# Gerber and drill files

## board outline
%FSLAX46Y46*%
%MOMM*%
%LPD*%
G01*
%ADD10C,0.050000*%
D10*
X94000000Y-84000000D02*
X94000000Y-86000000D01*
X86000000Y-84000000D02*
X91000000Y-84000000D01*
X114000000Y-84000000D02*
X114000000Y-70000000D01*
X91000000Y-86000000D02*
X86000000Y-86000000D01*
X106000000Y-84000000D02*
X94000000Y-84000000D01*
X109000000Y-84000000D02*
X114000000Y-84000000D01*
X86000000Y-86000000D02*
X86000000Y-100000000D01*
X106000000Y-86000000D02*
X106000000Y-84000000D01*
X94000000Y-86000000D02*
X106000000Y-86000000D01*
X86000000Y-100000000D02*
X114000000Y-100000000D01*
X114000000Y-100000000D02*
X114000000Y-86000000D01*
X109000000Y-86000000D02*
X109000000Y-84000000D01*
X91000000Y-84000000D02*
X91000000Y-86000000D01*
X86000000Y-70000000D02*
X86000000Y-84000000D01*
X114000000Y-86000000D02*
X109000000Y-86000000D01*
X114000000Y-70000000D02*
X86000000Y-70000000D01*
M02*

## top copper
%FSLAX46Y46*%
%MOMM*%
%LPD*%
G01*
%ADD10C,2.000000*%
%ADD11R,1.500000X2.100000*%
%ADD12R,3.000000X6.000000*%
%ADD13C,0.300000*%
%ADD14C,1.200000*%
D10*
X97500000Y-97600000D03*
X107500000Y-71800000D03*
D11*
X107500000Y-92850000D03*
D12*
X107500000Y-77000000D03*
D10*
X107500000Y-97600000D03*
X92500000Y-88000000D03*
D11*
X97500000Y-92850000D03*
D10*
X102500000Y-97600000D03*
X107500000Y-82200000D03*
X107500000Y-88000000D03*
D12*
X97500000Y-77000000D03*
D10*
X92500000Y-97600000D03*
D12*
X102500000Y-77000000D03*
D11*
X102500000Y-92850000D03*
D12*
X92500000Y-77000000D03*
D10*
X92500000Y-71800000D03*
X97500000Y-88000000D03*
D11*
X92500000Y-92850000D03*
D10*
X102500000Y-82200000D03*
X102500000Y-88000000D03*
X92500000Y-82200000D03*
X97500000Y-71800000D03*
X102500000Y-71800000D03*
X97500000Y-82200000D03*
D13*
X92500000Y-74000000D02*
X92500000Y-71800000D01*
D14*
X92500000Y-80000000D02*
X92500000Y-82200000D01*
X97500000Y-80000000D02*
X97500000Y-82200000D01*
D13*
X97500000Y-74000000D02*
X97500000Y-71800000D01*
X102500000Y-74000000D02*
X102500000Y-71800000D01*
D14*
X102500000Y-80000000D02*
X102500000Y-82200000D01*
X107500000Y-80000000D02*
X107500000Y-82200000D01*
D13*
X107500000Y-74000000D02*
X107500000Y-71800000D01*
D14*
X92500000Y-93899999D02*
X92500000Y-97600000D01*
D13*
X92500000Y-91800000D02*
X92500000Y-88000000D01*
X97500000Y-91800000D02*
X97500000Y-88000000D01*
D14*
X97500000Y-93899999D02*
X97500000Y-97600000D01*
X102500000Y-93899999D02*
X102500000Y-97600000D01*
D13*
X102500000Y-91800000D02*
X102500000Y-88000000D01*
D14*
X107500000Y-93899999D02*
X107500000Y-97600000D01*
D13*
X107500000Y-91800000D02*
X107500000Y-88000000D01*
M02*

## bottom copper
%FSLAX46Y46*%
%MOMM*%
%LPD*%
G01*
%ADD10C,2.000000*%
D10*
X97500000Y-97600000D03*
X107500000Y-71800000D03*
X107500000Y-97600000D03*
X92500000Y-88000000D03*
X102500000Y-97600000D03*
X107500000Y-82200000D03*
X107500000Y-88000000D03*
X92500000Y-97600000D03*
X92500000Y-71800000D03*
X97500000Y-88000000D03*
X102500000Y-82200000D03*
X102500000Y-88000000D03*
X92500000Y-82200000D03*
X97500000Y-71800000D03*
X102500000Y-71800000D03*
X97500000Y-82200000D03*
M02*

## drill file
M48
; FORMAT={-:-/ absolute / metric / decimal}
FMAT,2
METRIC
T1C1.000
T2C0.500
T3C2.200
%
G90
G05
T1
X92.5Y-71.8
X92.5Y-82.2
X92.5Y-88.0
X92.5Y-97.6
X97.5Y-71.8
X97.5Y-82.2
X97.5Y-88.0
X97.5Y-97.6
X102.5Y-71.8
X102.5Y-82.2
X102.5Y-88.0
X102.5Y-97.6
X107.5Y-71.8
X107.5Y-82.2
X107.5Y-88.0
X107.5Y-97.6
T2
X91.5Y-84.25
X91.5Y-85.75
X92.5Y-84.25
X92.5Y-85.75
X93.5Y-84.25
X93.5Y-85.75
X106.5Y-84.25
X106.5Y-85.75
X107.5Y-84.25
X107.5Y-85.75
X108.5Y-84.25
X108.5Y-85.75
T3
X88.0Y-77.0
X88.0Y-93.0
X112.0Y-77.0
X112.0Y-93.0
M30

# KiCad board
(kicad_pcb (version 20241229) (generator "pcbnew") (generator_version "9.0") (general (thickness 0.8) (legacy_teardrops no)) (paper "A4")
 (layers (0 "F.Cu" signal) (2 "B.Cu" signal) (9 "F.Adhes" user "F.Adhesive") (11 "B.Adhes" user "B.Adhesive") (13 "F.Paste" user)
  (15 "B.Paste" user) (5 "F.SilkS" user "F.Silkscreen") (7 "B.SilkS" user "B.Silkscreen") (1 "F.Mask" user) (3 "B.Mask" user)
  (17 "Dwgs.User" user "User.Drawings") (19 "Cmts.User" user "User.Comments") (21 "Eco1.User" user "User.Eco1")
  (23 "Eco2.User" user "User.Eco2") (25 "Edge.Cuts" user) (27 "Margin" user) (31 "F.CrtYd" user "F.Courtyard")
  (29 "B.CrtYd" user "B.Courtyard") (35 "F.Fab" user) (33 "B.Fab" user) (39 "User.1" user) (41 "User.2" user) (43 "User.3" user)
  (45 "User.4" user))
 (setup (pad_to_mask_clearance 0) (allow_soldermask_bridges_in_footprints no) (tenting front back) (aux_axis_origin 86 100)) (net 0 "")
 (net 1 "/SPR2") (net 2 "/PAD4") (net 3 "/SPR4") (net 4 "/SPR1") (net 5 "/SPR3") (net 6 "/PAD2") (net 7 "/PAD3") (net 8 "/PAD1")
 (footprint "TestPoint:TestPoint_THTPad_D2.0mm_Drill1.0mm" (layer "F.Cu") (at 97.5 97.6)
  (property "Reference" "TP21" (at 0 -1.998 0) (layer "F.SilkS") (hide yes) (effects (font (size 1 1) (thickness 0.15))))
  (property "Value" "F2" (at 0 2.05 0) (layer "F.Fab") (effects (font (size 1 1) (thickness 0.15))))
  (pad "1" thru_hole circle (at 0 0) (size 2 2) (drill 1) (layers "*.Cu" "*.Mask") (remove_unused_layers no) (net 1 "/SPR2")))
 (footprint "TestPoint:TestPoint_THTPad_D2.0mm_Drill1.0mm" (layer "F.Cu") (at 107.5 71.8)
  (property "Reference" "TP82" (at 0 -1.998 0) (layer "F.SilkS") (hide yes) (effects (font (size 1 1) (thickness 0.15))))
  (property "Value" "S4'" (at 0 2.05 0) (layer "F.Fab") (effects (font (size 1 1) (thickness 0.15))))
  (pad "1" thru_hole circle (at 0 0) (size 2 2) (drill 1) (layers "*.Cu" "*.Mask") (remove_unused_layers no) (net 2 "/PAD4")))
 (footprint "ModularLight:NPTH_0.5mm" (layer "F.Cu") (at 106.5 84.25)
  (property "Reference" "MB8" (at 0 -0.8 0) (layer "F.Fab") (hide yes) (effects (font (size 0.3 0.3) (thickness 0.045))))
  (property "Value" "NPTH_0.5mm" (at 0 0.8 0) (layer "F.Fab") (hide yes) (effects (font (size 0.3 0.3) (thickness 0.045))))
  (pad "" np_thru_hole circle (at 0 0) (size 0.5 0.5) (drill 0.5) (layers "*.Cu" "*.Mask")))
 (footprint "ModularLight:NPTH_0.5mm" (layer "F.Cu") (at 91.5 84.25)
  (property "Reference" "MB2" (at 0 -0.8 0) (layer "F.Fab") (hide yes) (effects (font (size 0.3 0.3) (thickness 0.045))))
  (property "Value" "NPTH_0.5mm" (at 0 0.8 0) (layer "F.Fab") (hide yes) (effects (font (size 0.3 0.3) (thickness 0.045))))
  (pad "" np_thru_hole circle (at 0 0) (size 0.5 0.5) (drill 0.5) (layers "*.Cu" "*.Mask")))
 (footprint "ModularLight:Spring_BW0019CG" (layer "F.Cu") (at 107.5 92.15)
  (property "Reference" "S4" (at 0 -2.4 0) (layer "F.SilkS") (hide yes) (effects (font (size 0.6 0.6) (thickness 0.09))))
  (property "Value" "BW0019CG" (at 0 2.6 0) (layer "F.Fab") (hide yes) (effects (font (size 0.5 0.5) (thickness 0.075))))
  (pad "1" smd rect (at 0 0.7) (size 1.5 2.1) (layers "F.Cu" "F.Mask" "F.Paste") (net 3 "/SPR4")))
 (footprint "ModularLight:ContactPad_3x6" (layer "F.Cu") (at 107.5 77)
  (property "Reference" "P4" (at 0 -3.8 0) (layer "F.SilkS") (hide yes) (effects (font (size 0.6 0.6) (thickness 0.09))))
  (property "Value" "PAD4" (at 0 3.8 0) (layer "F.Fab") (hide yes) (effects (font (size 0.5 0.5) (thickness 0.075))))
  (pad "1" smd rect (at 0 0) (size 3 6) (layers "F.Cu" "F.Mask") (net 2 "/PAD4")))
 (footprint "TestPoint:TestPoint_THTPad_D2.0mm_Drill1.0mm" (layer "F.Cu") (at 107.5 97.6)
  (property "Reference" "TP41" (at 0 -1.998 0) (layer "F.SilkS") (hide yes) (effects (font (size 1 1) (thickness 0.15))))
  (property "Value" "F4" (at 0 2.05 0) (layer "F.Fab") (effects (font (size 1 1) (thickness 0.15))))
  (pad "1" thru_hole circle (at 0 0) (size 2 2) (drill 1) (layers "*.Cu" "*.Mask") (remove_unused_layers no) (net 3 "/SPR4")))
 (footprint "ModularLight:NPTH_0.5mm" (layer "F.Cu") (at 93.5 84.25)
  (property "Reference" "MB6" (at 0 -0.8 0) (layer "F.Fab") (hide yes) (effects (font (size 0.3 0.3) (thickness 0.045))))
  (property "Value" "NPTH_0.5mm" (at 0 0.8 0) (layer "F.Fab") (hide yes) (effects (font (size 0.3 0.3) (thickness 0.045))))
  (pad "" np_thru_hole circle (at 0 0) (size 0.5 0.5) (drill 0.5) (layers "*.Cu" "*.Mask")))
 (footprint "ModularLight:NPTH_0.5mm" (layer "F.Cu") (at 108.5 85.75)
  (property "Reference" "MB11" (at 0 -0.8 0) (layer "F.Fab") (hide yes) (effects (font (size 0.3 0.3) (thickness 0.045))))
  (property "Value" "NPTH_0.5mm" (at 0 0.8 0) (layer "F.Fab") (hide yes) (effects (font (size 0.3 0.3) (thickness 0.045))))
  (pad "" np_thru_hole circle (at 0 0) (size 0.5 0.5) (drill 0.5) (layers "*.Cu" "*.Mask")))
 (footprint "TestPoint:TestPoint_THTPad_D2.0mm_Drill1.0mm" (layer "F.Cu") (at 92.5 88)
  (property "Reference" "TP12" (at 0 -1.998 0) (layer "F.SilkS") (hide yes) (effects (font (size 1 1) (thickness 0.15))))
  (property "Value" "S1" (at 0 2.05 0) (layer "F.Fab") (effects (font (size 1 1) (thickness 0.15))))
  (pad "1" thru_hole circle (at 0 0) (size 2 2) (drill 1) (layers "*.Cu" "*.Mask") (remove_unused_layers no) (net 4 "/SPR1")))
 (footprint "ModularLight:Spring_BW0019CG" (layer "F.Cu") (at 97.5 92.15)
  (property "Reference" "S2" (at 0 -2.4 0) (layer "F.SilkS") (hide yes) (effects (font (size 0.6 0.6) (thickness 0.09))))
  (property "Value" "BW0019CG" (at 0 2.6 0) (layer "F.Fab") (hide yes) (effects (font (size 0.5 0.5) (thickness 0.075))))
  (pad "1" smd rect (at 0 0.7) (size 1.5 2.1) (layers "F.Cu" "F.Mask" "F.Paste") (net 1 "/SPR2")))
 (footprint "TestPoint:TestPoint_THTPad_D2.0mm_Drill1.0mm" (layer "F.Cu") (at 102.5 97.6)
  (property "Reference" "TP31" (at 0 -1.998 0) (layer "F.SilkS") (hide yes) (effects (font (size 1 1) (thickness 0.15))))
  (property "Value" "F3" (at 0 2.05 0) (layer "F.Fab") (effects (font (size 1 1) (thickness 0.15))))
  (pad "1" thru_hole circle (at 0 0) (size 2 2) (drill 1) (layers "*.Cu" "*.Mask") (remove_unused_layers no) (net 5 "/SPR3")))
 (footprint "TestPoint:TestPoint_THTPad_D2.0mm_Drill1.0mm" (layer "F.Cu") (at 107.5 82.2)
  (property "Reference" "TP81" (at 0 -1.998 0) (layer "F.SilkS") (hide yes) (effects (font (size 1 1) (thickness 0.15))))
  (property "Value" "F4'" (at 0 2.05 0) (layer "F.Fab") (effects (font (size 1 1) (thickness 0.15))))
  (pad "1" thru_hole circle (at 0 0) (size 2 2) (drill 1) (layers "*.Cu" "*.Mask") (remove_unused_layers no) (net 2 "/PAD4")))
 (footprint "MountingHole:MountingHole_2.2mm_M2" (layer "F.Cu") (at 112 77)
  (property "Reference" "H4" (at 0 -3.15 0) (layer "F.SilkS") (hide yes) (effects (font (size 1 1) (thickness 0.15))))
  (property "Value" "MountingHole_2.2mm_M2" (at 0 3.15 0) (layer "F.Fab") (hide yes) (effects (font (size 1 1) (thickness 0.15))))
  (pad "" np_thru_hole circle (at 0 0) (size 2.2 2.2) (drill 2.2) (layers "*.Cu" "*.Mask")))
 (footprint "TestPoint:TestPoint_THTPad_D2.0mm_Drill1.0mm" (layer "F.Cu") (at 107.5 88)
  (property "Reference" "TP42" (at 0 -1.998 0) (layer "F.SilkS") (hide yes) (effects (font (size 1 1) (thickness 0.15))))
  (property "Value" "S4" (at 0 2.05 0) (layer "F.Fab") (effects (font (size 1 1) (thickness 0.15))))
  (pad "1" thru_hole circle (at 0 0) (size 2 2) (drill 1) (layers "*.Cu" "*.Mask") (remove_unused_layers no) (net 3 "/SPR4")))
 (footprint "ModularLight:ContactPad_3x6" (layer "F.Cu") (at 97.5 77)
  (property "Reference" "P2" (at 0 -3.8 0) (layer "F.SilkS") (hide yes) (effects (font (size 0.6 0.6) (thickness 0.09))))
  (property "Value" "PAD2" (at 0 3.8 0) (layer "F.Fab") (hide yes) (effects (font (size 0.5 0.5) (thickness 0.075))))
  (pad "1" smd rect (at 0 0) (size 3 6) (layers "F.Cu" "F.Mask") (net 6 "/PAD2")))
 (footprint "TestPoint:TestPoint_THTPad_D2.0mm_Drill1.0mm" (layer "F.Cu") (at 92.5 97.6)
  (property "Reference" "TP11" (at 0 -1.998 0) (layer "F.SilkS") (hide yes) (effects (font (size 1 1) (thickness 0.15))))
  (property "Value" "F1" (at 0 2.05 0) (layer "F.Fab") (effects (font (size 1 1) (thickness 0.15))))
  (pad "1" thru_hole circle (at 0 0) (size 2 2) (drill 1) (layers "*.Cu" "*.Mask") (remove_unused_layers no) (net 4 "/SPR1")))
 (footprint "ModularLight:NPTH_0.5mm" (layer "F.Cu") (at 106.5 85.75)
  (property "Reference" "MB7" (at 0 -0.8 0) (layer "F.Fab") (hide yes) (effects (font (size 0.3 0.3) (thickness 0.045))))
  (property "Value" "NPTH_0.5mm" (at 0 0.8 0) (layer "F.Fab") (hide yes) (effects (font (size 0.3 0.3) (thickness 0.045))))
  (pad "" np_thru_hole circle (at 0 0) (size 0.5 0.5) (drill 0.5) (layers "*.Cu" "*.Mask")))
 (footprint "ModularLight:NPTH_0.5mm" (layer "F.Cu") (at 91.5 85.75)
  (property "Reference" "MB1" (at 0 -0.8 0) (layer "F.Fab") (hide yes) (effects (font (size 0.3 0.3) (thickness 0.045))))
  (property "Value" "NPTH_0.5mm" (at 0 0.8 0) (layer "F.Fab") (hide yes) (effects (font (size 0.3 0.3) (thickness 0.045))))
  (pad "" np_thru_hole circle (at 0 0) (size 0.5 0.5) (drill 0.5) (layers "*.Cu" "*.Mask")))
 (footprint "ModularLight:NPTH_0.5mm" (layer "F.Cu") (at 107.5 85.75)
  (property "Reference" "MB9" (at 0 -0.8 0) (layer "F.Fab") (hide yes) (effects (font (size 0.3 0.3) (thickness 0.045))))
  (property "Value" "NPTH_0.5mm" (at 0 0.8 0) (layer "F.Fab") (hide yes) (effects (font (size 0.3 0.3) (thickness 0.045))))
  (pad "" np_thru_hole circle (at 0 0) (size 0.5 0.5) (drill 0.5) (layers "*.Cu" "*.Mask")))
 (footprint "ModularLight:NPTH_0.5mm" (layer "F.Cu") (at 108.5 84.25)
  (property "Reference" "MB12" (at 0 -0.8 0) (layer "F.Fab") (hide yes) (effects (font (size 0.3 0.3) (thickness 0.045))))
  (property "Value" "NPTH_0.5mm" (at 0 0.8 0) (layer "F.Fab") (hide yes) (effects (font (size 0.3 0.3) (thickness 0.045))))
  (pad "" np_thru_hole circle (at 0 0) (size 0.5 0.5) (drill 0.5) (layers "*.Cu" "*.Mask")))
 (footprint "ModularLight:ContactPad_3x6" (layer "F.Cu") (at 102.5 77)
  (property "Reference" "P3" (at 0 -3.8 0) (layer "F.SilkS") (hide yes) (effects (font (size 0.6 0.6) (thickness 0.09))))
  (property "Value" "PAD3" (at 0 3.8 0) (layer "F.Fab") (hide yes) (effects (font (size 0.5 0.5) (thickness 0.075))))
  (pad "1" smd rect (at 0 0) (size 3 6) (layers "F.Cu" "F.Mask") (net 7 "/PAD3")))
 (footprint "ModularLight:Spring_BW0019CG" (layer "F.Cu") (at 102.5 92.15)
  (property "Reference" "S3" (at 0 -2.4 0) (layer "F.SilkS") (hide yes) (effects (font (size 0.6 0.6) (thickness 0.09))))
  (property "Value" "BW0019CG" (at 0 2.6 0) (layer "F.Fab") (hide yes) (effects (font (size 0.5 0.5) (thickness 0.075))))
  (pad "1" smd rect (at 0 0.7) (size 1.5 2.1) (layers "F.Cu" "F.Mask" "F.Paste") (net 5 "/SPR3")))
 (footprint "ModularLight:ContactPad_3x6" (layer "F.Cu") (at 92.5 77)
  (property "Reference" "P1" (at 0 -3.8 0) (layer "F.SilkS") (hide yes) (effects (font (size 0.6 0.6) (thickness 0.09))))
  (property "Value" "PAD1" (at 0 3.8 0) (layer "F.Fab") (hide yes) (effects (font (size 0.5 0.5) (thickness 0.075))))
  (pad "1" smd rect (at 0 0) (size 3 6) (layers "F.Cu" "F.Mask") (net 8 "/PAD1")))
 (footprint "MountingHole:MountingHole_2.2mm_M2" (layer "F.Cu") (at 112 93)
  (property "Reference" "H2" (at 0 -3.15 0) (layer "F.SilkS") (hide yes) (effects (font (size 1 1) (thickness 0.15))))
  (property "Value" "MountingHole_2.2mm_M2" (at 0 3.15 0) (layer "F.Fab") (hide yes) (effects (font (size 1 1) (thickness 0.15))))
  (pad "" np_thru_hole circle (at 0 0) (size 2.2 2.2) (drill 2.2) (layers "*.Cu" "*.Mask")))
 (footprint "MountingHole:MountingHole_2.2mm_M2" (layer "F.Cu") (at 88 93)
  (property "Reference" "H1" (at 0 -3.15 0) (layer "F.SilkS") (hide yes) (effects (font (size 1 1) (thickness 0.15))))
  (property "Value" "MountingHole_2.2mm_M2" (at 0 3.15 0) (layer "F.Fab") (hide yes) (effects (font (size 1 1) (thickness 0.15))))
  (pad "" np_thru_hole circle (at 0 0) (size 2.2 2.2) (drill 2.2) (layers "*.Cu" "*.Mask")))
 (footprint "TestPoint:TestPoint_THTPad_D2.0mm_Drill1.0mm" (layer "F.Cu") (at 92.5 71.8)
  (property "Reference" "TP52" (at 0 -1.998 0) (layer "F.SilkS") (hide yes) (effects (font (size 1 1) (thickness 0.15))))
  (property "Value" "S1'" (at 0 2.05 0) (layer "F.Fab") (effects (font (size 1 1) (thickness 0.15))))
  (pad "1" thru_hole circle (at 0 0) (size 2 2) (drill 1) (layers "*.Cu" "*.Mask") (remove_unused_layers no) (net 8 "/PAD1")))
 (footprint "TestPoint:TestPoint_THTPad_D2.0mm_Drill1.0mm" (layer "F.Cu") (at 97.5 88)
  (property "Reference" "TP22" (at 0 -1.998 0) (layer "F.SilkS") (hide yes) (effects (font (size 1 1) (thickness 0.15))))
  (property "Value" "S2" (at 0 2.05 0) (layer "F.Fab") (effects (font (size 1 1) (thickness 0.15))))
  (pad "1" thru_hole circle (at 0 0) (size 2 2) (drill 1) (layers "*.Cu" "*.Mask") (remove_unused_layers no) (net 1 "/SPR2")))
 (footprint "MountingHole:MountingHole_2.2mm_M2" (layer "F.Cu") (at 88 77)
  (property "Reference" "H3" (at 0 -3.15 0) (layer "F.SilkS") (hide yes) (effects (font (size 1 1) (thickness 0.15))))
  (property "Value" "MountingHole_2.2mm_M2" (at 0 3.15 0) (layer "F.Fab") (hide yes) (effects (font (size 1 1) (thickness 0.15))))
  (pad "" np_thru_hole circle (at 0 0) (size 2.2 2.2) (drill 2.2) (layers "*.Cu" "*.Mask")))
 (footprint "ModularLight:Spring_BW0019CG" (layer "F.Cu") (at 92.5 92.15)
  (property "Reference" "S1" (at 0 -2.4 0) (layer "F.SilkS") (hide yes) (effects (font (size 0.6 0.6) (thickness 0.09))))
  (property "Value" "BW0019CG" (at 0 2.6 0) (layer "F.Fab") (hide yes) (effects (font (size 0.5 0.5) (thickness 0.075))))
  (pad "1" smd rect (at 0 0.7) (size 1.5 2.1) (layers "F.Cu" "F.Mask" "F.Paste") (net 4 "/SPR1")))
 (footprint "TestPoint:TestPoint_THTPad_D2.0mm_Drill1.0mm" (layer "F.Cu") (at 102.5 82.2)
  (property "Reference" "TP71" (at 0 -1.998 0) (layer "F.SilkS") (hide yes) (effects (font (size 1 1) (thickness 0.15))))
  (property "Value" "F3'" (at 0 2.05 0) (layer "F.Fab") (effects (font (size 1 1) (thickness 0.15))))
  (pad "1" thru_hole circle (at 0 0) (size 2 2) (drill 1) (layers "*.Cu" "*.Mask") (remove_unused_layers no) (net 7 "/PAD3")))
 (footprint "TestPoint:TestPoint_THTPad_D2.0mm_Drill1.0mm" (layer "F.Cu") (at 102.5 88)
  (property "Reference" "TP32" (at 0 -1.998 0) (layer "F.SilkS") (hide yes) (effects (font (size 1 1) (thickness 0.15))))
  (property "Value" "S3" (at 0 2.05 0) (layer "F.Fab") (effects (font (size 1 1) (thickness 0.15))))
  (pad "1" thru_hole circle (at 0 0) (size 2 2) (drill 1) (layers "*.Cu" "*.Mask") (remove_unused_layers no) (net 5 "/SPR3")))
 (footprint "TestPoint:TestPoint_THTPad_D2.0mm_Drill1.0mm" (layer "F.Cu") (at 92.5 82.2)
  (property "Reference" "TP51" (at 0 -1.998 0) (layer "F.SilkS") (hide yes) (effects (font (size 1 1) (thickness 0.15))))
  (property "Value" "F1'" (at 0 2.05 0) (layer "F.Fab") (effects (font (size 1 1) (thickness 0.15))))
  (pad "1" thru_hole circle (at 0 0) (size 2 2) (drill 1) (layers "*.Cu" "*.Mask") (remove_unused_layers no) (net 8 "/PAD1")))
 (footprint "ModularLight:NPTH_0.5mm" (layer "F.Cu") (at 92.5 84.25)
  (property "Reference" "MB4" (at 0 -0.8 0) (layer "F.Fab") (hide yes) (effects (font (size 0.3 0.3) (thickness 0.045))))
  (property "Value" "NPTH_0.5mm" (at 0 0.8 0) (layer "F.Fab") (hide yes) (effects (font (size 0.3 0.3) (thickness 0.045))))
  (pad "" np_thru_hole circle (at 0 0) (size 0.5 0.5) (drill 0.5) (layers "*.Cu" "*.Mask")))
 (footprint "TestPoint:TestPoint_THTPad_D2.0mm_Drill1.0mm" (layer "F.Cu") (at 97.5 71.8)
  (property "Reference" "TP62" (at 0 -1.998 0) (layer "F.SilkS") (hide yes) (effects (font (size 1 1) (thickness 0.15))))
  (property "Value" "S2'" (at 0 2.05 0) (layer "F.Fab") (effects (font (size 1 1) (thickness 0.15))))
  (pad "1" thru_hole circle (at 0 0) (size 2 2) (drill 1) (layers "*.Cu" "*.Mask") (remove_unused_layers no) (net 6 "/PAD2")))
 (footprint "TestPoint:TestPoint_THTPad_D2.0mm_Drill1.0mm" (layer "F.Cu") (at 102.5 71.8)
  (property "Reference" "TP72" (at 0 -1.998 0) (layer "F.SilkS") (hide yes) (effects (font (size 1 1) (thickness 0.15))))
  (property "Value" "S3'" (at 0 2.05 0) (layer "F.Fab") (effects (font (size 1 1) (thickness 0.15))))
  (pad "1" thru_hole circle (at 0 0) (size 2 2) (drill 1) (layers "*.Cu" "*.Mask") (remove_unused_layers no) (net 7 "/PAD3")))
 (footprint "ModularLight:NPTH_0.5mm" (layer "F.Cu") (at 93.5 85.75)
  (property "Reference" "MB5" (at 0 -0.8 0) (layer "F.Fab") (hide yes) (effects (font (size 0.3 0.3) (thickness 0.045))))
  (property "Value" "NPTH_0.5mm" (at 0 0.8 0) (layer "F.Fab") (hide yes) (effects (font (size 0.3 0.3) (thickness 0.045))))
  (pad "" np_thru_hole circle (at 0 0) (size 0.5 0.5) (drill 0.5) (layers "*.Cu" "*.Mask")))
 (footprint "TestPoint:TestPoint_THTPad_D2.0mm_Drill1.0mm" (layer "F.Cu") (at 97.5 82.2)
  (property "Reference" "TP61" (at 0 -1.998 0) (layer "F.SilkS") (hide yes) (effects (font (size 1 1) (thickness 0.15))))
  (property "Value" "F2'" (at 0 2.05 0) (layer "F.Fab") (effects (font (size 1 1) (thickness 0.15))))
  (pad "1" thru_hole circle (at 0 0) (size 2 2) (drill 1) (layers "*.Cu" "*.Mask") (remove_unused_layers no) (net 6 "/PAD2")))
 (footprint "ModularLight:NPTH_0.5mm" (layer "F.Cu") (at 107.5 84.25)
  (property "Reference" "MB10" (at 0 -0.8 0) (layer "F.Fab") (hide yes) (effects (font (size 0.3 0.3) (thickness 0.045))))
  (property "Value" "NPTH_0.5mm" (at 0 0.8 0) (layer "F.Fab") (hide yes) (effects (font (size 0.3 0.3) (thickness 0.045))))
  (pad "" np_thru_hole circle (at 0 0) (size 0.5 0.5) (drill 0.5) (layers "*.Cu" "*.Mask")))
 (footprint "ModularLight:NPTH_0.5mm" (layer "F.Cu") (at 92.5 85.75)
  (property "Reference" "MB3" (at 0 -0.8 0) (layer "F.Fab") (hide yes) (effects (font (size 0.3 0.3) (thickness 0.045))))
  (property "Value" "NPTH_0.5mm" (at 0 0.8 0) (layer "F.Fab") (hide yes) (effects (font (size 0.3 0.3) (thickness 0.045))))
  (pad "" np_thru_hole circle (at 0 0) (size 0.5 0.5) (drill 0.5) (layers "*.Cu" "*.Mask")))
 (gr_line (start 94 84) (end 94 86) (stroke (width 0.05) (type default)) (layer "Edge.Cuts"))
 (gr_line (start 86 84) (end 91 84) (stroke (width 0.05) (type default)) (layer "Edge.Cuts"))
 (gr_line (start 114 84) (end 114 70) (stroke (width 0.05) (type default)) (layer "Edge.Cuts"))
 (gr_line (start 91 86) (end 86 86) (stroke (width 0.05) (type default)) (layer "Edge.Cuts"))
 (gr_line (start 106 84) (end 94 84) (stroke (width 0.05) (type default)) (layer "Edge.Cuts"))
 (gr_line (start 109 84) (end 114 84) (stroke (width 0.05) (type default)) (layer "Edge.Cuts"))
 (gr_line (start 86 86) (end 86 100) (stroke (width 0.05) (type default)) (layer "Edge.Cuts"))
 (gr_line (start 106 86) (end 106 84) (stroke (width 0.05) (type default)) (layer "Edge.Cuts"))
 (gr_line (start 94 86) (end 106 86) (stroke (width 0.05) (type default)) (layer "Edge.Cuts"))
 (gr_line (start 86 100) (end 114 100) (stroke (width 0.05) (type default)) (layer "Edge.Cuts"))
 (gr_line (start 114 100) (end 114 86) (stroke (width 0.05) (type default)) (layer "Edge.Cuts"))
 (gr_line (start 109 86) (end 109 84) (stroke (width 0.05) (type default)) (layer "Edge.Cuts"))
 (gr_line (start 91 84) (end 91 86) (stroke (width 0.05) (type default)) (layer "Edge.Cuts"))
 (gr_line (start 86 70) (end 86 84) (stroke (width 0.05) (type default)) (layer "Edge.Cuts"))
 (gr_line (start 114 86) (end 109 86) (stroke (width 0.05) (type default)) (layer "Edge.Cuts"))
 (gr_line (start 114 70) (end 86 70) (stroke (width 0.05) (type default)) (layer "Edge.Cuts"))
 (segment (start 92.5 74) (end 92.5 71.8) (width 0.3) (locked yes) (layer "F.Cu") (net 8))
 (segment (start 92.5 80) (end 92.5 82.2) (width 1.2) (locked yes) (layer "F.Cu") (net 8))
 (segment (start 97.5 80) (end 97.5 82.2) (width 1.2) (locked yes) (layer "F.Cu") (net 6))
 (segment (start 97.5 74) (end 97.5 71.8) (width 0.3) (locked yes) (layer "F.Cu") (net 6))
 (segment (start 102.5 74) (end 102.5 71.8) (width 0.3) (locked yes) (layer "F.Cu") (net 7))
 (segment (start 102.5 80) (end 102.5 82.2) (width 1.2) (locked yes) (layer "F.Cu") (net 7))
 (segment (start 107.5 80) (end 107.5 82.2) (width 1.2) (locked yes) (layer "F.Cu") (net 2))
 (segment (start 107.5 74) (end 107.5 71.8) (width 0.3) (locked yes) (layer "F.Cu") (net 2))
 (segment (start 92.5 93.899999) (end 92.5 97.6) (width 1.2) (locked yes) (layer "F.Cu") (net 4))
 (segment (start 92.5 91.8) (end 92.5 88) (width 0.3) (locked yes) (layer "F.Cu") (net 4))
 (segment (start 97.5 91.8) (end 97.5 88) (width 0.3) (locked yes) (layer "F.Cu") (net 1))
 (segment (start 97.5 93.899999) (end 97.5 97.6) (width 1.2) (locked yes) (layer "F.Cu") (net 1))
 (segment (start 102.5 93.899999) (end 102.5 97.6) (width 1.2) (locked yes) (layer "F.Cu") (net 5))
 (segment (start 102.5 91.8) (end 102.5 88) (width 0.3) (locked yes) (layer "F.Cu") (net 5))
 (segment (start 107.5 93.899999) (end 107.5 97.6) (width 1.2) (locked yes) (layer "F.Cu") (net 3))
 (segment (start 107.5 91.8) (end 107.5 88) (width 0.3) (locked yes) (layer "F.Cu") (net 3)))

